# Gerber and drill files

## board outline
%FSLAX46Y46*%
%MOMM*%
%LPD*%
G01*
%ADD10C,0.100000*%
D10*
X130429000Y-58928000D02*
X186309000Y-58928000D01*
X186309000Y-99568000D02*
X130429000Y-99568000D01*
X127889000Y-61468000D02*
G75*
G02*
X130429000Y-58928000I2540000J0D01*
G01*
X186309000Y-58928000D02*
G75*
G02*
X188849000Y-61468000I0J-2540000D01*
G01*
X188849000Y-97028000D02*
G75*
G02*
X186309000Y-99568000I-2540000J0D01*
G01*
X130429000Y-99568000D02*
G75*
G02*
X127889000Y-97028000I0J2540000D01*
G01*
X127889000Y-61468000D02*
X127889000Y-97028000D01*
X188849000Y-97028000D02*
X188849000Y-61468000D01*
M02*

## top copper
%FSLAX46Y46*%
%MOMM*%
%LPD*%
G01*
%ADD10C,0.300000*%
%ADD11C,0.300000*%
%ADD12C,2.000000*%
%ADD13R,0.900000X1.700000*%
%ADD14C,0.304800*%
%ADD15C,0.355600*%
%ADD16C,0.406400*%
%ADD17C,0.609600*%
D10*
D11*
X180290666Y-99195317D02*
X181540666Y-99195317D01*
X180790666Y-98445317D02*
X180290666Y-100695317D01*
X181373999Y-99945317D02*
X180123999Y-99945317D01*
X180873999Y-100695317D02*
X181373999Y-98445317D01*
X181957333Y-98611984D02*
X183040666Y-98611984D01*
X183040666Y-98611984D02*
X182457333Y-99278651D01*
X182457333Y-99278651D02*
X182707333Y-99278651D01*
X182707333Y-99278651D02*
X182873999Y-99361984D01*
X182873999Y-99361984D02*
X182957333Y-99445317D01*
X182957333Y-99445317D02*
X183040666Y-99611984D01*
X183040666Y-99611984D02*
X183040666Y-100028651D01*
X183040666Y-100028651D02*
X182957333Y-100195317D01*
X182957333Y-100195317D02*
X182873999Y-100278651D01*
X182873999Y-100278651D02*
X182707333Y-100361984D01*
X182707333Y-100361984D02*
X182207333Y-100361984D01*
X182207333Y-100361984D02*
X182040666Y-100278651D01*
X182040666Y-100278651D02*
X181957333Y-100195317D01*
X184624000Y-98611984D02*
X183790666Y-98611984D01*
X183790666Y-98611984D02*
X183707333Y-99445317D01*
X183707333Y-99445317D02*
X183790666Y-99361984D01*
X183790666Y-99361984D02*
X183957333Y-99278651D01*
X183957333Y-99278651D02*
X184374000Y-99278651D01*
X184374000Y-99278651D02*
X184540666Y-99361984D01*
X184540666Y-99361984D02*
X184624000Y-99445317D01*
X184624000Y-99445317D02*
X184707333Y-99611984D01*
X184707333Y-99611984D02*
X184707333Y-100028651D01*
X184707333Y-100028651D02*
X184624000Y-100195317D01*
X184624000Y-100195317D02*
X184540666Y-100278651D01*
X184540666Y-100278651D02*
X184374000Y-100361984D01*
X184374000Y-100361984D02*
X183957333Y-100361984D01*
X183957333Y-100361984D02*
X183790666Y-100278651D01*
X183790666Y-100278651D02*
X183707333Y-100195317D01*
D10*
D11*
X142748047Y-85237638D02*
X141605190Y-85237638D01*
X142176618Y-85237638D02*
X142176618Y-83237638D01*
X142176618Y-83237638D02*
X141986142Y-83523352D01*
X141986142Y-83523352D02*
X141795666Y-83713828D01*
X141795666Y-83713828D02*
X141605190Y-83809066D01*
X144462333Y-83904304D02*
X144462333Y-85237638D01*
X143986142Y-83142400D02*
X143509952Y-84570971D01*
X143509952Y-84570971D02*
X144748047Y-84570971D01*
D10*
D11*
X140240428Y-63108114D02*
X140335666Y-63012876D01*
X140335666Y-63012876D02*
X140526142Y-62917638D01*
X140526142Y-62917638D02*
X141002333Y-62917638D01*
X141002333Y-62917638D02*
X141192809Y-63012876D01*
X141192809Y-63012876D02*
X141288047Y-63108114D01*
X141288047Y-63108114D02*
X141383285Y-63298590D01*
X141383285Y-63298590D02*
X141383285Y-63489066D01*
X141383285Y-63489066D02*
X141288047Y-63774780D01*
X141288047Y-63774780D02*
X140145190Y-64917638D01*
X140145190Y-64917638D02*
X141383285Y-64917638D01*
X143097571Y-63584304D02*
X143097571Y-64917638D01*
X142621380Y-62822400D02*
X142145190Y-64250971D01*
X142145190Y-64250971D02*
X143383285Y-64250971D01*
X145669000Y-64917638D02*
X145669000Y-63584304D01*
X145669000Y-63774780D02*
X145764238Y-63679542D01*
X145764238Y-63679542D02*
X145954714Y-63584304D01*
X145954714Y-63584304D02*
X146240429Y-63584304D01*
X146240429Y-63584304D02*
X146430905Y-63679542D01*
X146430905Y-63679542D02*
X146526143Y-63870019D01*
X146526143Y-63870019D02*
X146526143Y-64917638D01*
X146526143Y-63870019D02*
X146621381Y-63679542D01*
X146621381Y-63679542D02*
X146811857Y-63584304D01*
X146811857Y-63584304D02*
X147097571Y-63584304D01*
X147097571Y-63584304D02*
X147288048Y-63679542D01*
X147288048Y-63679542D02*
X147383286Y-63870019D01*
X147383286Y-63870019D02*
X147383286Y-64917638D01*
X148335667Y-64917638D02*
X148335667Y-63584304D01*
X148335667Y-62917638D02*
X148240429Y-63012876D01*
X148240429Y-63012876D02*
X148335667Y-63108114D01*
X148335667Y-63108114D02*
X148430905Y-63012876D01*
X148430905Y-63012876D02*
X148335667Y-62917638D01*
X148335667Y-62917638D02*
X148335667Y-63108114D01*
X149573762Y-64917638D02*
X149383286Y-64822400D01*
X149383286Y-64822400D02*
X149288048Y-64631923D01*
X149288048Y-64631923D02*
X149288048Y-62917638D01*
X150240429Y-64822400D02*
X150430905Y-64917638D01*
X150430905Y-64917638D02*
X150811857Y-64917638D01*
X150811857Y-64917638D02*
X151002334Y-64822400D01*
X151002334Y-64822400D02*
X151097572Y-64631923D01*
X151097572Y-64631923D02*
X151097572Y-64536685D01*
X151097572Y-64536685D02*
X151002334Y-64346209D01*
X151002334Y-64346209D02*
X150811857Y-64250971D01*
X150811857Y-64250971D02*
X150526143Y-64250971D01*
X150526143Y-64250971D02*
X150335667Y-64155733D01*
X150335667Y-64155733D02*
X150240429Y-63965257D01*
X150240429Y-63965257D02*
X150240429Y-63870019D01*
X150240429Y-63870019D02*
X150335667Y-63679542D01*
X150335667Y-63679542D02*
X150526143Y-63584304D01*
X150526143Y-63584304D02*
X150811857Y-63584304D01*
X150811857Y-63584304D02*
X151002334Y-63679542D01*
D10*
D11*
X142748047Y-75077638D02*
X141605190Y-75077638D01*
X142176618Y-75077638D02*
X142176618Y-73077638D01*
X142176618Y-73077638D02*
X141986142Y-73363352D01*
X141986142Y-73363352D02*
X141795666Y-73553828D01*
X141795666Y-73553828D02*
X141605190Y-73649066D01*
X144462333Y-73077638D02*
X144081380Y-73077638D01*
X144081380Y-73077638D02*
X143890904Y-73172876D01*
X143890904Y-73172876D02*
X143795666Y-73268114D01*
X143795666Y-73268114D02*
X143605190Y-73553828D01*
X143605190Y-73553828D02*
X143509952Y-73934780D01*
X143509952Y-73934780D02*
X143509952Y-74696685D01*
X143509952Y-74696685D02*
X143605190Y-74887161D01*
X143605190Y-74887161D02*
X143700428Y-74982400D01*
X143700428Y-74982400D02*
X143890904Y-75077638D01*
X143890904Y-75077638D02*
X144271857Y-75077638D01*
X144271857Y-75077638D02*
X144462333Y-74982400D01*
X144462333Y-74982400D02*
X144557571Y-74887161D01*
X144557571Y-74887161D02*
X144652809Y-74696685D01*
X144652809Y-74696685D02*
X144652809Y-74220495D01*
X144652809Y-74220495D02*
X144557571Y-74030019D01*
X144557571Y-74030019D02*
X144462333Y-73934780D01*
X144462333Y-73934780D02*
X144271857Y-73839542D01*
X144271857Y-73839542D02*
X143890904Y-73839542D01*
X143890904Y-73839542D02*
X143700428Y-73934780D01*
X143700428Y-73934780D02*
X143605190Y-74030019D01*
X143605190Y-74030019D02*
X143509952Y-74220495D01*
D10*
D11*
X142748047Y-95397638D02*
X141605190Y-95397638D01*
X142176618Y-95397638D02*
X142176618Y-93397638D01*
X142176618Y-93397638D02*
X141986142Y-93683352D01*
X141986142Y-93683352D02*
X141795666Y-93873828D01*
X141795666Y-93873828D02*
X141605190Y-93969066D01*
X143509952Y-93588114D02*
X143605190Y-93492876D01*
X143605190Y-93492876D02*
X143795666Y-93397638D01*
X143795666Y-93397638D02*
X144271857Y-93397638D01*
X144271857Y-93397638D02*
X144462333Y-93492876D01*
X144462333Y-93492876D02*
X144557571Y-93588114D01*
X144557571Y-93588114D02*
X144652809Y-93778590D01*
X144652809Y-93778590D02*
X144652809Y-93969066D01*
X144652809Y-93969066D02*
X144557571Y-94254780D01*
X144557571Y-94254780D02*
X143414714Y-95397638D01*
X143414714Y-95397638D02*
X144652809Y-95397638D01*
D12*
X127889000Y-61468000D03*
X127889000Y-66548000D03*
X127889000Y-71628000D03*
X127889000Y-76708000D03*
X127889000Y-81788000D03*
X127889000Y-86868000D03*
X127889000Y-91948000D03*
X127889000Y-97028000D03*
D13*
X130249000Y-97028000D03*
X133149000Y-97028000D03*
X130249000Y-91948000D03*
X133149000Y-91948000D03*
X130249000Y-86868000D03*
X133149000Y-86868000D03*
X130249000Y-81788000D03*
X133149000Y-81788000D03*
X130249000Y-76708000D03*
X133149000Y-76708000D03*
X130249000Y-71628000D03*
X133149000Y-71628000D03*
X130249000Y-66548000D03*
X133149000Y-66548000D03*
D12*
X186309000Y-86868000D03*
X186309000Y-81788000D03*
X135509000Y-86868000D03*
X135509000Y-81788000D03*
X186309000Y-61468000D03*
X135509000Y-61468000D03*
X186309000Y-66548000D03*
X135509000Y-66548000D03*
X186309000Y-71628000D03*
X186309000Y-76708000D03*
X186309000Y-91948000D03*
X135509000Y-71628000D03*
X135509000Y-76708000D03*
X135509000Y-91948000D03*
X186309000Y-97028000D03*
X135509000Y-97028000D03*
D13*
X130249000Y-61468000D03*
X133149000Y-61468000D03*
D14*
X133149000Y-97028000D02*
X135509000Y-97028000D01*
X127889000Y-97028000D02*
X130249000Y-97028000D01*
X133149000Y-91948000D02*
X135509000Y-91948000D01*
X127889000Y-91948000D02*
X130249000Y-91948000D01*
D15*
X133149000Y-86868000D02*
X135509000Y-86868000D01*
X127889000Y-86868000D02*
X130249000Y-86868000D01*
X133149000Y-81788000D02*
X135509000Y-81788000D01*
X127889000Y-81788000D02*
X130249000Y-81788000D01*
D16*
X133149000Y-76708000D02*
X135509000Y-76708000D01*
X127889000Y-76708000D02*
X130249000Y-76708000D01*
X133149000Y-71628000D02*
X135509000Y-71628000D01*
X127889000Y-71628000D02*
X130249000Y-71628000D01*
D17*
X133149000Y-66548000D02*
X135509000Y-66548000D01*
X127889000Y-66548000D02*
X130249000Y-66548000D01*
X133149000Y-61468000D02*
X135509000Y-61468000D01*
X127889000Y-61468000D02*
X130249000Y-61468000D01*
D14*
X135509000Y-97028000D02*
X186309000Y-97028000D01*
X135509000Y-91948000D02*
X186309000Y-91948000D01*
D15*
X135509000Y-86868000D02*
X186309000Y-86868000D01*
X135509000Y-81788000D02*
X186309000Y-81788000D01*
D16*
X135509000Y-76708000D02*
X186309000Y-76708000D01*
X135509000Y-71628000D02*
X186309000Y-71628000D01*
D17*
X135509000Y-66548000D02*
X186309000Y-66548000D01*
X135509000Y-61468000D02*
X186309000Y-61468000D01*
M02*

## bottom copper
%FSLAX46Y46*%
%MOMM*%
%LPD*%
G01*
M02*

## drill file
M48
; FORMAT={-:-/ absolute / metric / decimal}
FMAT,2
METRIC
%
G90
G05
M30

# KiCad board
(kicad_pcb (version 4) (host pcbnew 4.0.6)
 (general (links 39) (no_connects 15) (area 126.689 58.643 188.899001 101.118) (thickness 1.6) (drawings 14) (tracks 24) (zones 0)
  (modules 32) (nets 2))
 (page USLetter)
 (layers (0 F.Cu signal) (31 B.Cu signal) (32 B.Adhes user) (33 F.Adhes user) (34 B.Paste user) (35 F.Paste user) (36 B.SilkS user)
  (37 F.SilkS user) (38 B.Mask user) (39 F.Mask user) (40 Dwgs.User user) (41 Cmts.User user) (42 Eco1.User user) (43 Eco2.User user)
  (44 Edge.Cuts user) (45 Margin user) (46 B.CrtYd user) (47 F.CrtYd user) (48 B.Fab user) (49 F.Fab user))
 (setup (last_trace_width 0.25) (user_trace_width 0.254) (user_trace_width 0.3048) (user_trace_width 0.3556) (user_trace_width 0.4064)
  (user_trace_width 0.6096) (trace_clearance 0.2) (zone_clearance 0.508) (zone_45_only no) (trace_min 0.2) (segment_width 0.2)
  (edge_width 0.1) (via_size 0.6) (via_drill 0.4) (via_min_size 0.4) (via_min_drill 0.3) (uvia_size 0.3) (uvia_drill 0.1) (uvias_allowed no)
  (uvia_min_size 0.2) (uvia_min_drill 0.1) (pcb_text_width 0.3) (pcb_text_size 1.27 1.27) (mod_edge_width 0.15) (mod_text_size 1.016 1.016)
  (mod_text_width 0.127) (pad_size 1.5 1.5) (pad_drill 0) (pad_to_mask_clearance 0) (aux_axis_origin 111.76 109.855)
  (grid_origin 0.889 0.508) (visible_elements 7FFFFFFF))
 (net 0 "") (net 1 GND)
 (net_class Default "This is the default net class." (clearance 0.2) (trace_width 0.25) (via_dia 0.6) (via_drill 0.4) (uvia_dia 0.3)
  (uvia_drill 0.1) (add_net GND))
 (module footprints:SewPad (layer F.Cu) (at 127.889 61.468 90)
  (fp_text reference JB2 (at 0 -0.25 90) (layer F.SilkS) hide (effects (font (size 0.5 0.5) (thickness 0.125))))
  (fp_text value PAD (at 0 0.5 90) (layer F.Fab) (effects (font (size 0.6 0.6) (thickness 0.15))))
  (pad 1 smd circle (at 0 0 90) (size 2 2) (layers F.Cu F.Mask) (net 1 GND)))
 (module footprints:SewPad (layer F.Cu) (at 127.889 66.548 90)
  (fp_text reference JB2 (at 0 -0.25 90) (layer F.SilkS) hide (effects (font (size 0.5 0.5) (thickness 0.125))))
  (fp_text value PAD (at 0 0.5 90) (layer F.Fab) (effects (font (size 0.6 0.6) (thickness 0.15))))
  (pad 1 smd circle (at 0 0 90) (size 2 2) (layers F.Cu F.Mask) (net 1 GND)))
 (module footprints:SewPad (layer F.Cu) (at 127.889 71.628 90)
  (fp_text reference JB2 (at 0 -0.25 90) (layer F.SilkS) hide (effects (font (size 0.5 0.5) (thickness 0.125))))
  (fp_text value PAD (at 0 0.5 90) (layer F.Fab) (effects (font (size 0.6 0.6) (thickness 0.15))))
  (pad 1 smd circle (at 0 0 90) (size 2 2) (layers F.Cu F.Mask) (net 1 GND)))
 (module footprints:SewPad (layer F.Cu) (at 127.889 76.708 90)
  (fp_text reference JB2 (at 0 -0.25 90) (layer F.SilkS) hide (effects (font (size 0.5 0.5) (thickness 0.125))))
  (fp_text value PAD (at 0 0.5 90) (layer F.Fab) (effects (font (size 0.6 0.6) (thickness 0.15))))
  (pad 1 smd circle (at 0 0 90) (size 2 2) (layers F.Cu F.Mask) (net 1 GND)))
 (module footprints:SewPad (layer F.Cu) (at 127.889 81.788 90)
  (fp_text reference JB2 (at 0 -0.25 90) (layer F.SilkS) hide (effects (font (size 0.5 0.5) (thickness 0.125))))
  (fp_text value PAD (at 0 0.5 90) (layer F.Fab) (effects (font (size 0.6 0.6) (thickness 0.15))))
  (pad 1 smd circle (at 0 0 90) (size 2 2) (layers F.Cu F.Mask) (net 1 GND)))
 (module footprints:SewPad (layer F.Cu) (at 127.889 86.868 90)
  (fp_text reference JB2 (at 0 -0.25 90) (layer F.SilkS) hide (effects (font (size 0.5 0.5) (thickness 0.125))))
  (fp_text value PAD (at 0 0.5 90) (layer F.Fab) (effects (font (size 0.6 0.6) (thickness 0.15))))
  (pad 1 smd circle (at 0 0 90) (size 2 2) (layers F.Cu F.Mask) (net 1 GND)))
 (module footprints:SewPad (layer F.Cu) (at 127.889 91.948 90)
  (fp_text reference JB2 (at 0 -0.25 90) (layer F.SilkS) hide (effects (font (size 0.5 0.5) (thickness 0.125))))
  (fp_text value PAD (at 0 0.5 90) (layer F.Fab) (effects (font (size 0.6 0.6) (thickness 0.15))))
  (pad 1 smd circle (at 0 0 90) (size 2 2) (layers F.Cu F.Mask) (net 1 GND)))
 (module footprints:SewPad (layer F.Cu) (at 127.889 97.028 90)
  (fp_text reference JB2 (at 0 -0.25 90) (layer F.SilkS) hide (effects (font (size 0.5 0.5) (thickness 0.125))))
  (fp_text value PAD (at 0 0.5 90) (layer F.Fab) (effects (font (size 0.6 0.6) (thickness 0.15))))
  (pad 1 smd circle (at 0 0 90) (size 2 2) (layers F.Cu F.Mask) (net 1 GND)))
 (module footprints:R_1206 (layer F.Cu) (at 131.699 97.028)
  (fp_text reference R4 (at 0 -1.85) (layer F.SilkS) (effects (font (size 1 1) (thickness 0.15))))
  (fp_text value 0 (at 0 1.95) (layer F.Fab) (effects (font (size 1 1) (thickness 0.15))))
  (pad 1 smd rect (at -1.45 0) (size 0.9 1.7) (layers F.Cu F.Paste F.Mask) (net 1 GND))
  (pad 2 smd rect (at 1.45 0) (size 0.9 1.7) (layers F.Cu F.Paste F.Mask) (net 1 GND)))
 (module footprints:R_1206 (layer F.Cu) (at 131.699 91.948)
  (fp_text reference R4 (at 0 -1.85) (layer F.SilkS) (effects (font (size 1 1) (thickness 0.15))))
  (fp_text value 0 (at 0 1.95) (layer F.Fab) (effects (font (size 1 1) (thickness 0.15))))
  (pad 1 smd rect (at -1.45 0) (size 0.9 1.7) (layers F.Cu F.Paste F.Mask) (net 1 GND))
  (pad 2 smd rect (at 1.45 0) (size 0.9 1.7) (layers F.Cu F.Paste F.Mask) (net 1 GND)))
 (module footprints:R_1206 (layer F.Cu) (at 131.699 86.868)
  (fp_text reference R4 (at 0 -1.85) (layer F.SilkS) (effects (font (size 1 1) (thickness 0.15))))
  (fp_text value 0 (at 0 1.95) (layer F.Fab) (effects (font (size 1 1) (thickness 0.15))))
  (pad 1 smd rect (at -1.45 0) (size 0.9 1.7) (layers F.Cu F.Paste F.Mask) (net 1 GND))
  (pad 2 smd rect (at 1.45 0) (size 0.9 1.7) (layers F.Cu F.Paste F.Mask) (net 1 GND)))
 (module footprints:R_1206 (layer F.Cu) (at 131.699 81.788)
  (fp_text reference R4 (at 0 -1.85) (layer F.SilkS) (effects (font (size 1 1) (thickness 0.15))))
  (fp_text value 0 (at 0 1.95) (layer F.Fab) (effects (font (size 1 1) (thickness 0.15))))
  (pad 1 smd rect (at -1.45 0) (size 0.9 1.7) (layers F.Cu F.Paste F.Mask) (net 1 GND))
  (pad 2 smd rect (at 1.45 0) (size 0.9 1.7) (layers F.Cu F.Paste F.Mask) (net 1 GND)))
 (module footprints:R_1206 (layer F.Cu) (at 131.699 76.708)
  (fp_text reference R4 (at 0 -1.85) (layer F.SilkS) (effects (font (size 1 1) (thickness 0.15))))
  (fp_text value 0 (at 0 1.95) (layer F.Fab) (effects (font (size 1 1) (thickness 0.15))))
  (pad 1 smd rect (at -1.45 0) (size 0.9 1.7) (layers F.Cu F.Paste F.Mask) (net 1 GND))
  (pad 2 smd rect (at 1.45 0) (size 0.9 1.7) (layers F.Cu F.Paste F.Mask) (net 1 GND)))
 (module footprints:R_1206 (layer F.Cu) (at 131.699 71.628)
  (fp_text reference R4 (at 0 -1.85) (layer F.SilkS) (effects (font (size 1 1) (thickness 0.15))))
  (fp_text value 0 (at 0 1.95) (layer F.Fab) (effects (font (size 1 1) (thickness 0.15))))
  (pad 1 smd rect (at -1.45 0) (size 0.9 1.7) (layers F.Cu F.Paste F.Mask) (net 1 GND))
  (pad 2 smd rect (at 1.45 0) (size 0.9 1.7) (layers F.Cu F.Paste F.Mask) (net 1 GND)))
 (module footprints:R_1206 (layer F.Cu) (at 131.699 66.548)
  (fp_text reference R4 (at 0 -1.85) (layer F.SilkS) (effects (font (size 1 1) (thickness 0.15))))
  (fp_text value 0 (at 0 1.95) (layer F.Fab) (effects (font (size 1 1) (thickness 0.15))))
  (pad 1 smd rect (at -1.45 0) (size 0.9 1.7) (layers F.Cu F.Paste F.Mask) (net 1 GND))
  (pad 2 smd rect (at 1.45 0) (size 0.9 1.7) (layers F.Cu F.Paste F.Mask) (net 1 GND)))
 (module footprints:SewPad (layer F.Cu) (at 186.309 86.868 90)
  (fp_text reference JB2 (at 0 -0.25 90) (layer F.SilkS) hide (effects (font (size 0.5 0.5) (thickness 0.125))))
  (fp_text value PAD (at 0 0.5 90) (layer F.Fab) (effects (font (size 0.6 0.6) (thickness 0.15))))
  (pad 1 smd circle (at 0 0 90) (size 2 2) (layers F.Cu F.Mask) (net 1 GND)))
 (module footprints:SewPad (layer F.Cu) (at 186.309 81.788 90)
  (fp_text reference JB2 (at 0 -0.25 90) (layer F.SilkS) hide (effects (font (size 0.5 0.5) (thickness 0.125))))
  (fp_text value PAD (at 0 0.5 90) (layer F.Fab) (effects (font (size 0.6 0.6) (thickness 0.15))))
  (pad 1 smd circle (at 0 0 90) (size 2 2) (layers F.Cu F.Mask) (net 1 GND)))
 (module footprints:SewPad (layer F.Cu) (at 135.509 86.868 90)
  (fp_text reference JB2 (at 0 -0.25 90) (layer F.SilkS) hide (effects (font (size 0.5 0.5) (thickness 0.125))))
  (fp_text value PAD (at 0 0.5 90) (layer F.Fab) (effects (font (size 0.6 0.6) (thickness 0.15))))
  (pad 1 smd circle (at 0 0 90) (size 2 2) (layers F.Cu F.Mask) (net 1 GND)))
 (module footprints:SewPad (layer F.Cu) (at 135.509 81.788 90)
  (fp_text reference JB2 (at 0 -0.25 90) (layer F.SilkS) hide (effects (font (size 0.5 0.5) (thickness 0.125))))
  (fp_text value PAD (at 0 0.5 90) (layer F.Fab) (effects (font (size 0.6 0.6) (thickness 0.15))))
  (pad 1 smd circle (at 0 0 90) (size 2 2) (layers F.Cu F.Mask) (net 1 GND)))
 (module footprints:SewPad (layer F.Cu) (at 186.309 61.468 90)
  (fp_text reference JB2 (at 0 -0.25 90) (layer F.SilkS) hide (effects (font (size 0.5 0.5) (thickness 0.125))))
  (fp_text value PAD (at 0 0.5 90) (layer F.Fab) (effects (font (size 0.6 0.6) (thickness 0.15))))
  (pad 1 smd circle (at 0 0 90) (size 2 2) (layers F.Cu F.Mask) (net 1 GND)))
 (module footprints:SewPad (layer F.Cu) (at 135.509 61.468 90)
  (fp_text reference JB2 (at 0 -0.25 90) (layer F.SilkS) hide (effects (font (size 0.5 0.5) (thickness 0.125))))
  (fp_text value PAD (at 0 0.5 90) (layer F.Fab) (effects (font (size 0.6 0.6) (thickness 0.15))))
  (pad 1 smd circle (at 0 0 90) (size 2 2) (layers F.Cu F.Mask) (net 1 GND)))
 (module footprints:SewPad (layer F.Cu) (at 186.309 66.548 90)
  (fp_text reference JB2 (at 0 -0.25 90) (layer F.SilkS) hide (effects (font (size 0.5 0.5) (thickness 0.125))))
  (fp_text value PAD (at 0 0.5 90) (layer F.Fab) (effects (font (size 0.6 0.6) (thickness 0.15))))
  (pad 1 smd circle (at 0 0 90) (size 2 2) (layers F.Cu F.Mask) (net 1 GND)))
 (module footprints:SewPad (layer F.Cu) (at 135.509 66.548 90)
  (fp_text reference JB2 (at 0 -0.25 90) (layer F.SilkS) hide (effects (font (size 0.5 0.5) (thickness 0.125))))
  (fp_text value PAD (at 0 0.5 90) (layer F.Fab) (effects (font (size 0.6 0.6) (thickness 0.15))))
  (pad 1 smd circle (at 0 0 90) (size 2 2) (layers F.Cu F.Mask) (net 1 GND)))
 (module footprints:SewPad (layer F.Cu) (at 186.309 71.628 90)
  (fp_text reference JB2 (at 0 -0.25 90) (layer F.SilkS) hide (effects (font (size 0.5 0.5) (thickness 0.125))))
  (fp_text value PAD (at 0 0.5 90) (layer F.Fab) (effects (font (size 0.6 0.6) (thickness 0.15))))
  (pad 1 smd circle (at 0 0 90) (size 2 2) (layers F.Cu F.Mask) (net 1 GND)))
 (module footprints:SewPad (layer F.Cu) (at 186.309 76.708 90)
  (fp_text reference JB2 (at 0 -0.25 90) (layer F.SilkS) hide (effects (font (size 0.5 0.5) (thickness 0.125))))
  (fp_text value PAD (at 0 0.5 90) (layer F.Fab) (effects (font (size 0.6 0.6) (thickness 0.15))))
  (pad 1 smd circle (at 0 0 90) (size 2 2) (layers F.Cu F.Mask) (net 1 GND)))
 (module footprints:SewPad (layer F.Cu) (at 186.309 91.948 90)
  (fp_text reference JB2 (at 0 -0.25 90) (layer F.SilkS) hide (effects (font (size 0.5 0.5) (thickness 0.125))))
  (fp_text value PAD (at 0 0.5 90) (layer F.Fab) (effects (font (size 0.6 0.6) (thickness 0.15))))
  (pad 1 smd circle (at 0 0 90) (size 2 2) (layers F.Cu F.Mask) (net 1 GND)))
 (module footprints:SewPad (layer F.Cu) (at 135.509 71.628 90)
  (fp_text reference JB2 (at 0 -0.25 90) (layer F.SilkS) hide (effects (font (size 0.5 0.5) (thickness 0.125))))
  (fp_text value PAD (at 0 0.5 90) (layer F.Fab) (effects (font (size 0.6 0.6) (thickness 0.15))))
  (pad 1 smd circle (at 0 0 90) (size 2 2) (layers F.Cu F.Mask) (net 1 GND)))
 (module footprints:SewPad (layer F.Cu) (at 135.509 76.708 90)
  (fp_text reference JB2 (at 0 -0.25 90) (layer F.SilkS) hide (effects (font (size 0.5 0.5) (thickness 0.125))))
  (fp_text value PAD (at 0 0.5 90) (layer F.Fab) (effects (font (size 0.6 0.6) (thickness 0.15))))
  (pad 1 smd circle (at 0 0 90) (size 2 2) (layers F.Cu F.Mask) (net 1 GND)))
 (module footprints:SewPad (layer F.Cu) (at 135.509 91.948 90)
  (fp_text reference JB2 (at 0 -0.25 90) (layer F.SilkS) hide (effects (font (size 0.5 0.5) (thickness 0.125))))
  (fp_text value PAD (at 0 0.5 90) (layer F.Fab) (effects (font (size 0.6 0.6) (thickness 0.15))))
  (pad 1 smd circle (at 0 0 90) (size 2 2) (layers F.Cu F.Mask) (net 1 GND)))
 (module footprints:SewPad (layer F.Cu) (at 186.309 97.028 90)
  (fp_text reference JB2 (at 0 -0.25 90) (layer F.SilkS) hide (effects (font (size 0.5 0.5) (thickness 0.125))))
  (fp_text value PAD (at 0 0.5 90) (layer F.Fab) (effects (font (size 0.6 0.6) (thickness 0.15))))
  (pad 1 smd circle (at 0 0 90) (size 2 2) (layers F.Cu F.Mask) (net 1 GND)))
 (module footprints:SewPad (layer F.Cu) (at 135.509 97.028 90)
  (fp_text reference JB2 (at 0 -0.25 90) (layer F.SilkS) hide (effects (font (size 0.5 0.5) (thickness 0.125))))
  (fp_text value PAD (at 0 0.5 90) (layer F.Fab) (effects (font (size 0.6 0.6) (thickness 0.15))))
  (pad 1 smd circle (at 0 0 90) (size 2 2) (layers F.Cu F.Mask) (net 1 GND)))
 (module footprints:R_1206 (layer F.Cu) (at 131.699 61.468)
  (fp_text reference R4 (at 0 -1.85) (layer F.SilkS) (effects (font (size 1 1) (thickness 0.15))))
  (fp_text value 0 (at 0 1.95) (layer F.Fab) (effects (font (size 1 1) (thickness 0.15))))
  (pad 1 smd rect (at -1.45 0) (size 0.9 1.7) (layers F.Cu F.Paste F.Mask) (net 1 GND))
  (pad 2 smd rect (at 1.45 0) (size 0.9 1.7) (layers F.Cu F.Paste F.Mask) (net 1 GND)))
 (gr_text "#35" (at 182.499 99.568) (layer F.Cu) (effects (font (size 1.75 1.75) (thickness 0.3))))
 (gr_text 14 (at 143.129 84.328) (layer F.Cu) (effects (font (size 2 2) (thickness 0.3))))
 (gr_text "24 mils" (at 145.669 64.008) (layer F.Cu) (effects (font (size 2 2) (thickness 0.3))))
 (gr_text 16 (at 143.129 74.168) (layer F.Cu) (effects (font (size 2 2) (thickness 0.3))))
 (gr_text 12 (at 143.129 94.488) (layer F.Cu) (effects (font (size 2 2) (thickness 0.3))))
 (gr_line (start 130.429 58.928) (end 186.309 58.928) (angle 90) (layer Edge.Cuts) (width 0.1))
 (gr_line (start 186.309 99.568) (end 130.429 99.568) (angle 90) (layer Edge.Cuts) (width 0.1))
 (gr_arc (start 130.429 61.468) (end 127.889 61.468) (angle 90) (layer Edge.Cuts) (width 0.1))
 (gr_arc (start 186.309 61.468) (end 186.309 58.928) (angle 90) (layer Edge.Cuts) (width 0.1))
 (gr_arc (start 186.309 97.028) (end 188.849 97.028) (angle 90) (layer Edge.Cuts) (width 0.1))
 (gr_arc (start 130.429 97.028) (end 130.429 99.568) (angle 90) (layer Edge.Cuts) (width 0.1))
 (gr_line (start 127.889 61.468) (end 127.889 97.028) (angle 90) (layer Edge.Cuts) (width 0.1))
 (gr_line (start 188.849 97.028) (end 188.849 61.468) (angle 90) (layer Edge.Cuts) (width 0.1))
 (segment (start 133.149 97.028) (end 135.509 97.028) (width 0.3048) (layer F.Cu) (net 1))
 (segment (start 127.889 97.028) (end 130.249 97.028) (width 0.3048) (layer F.Cu) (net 1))
 (segment (start 133.149 91.948) (end 135.509 91.948) (width 0.3048) (layer F.Cu) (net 1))
 (segment (start 127.889 91.948) (end 130.249 91.948) (width 0.3048) (layer F.Cu) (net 1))
 (segment (start 133.149 86.868) (end 135.509 86.868) (width 0.3556) (layer F.Cu) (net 1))
 (segment (start 127.889 86.868) (end 130.249 86.868) (width 0.3556) (layer F.Cu) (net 1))
 (segment (start 133.149 81.788) (end 135.509 81.788) (width 0.3556) (layer F.Cu) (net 1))
 (segment (start 127.889 81.788) (end 130.249 81.788) (width 0.3556) (layer F.Cu) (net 1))
 (segment (start 133.149 76.708) (end 135.509 76.708) (width 0.4064) (layer F.Cu) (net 1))
 (segment (start 127.889 76.708) (end 130.249 76.708) (width 0.4064) (layer F.Cu) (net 1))
 (segment (start 133.149 71.628) (end 135.509 71.628) (width 0.4064) (layer F.Cu) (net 1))
 (segment (start 127.889 71.628) (end 130.249 71.628) (width 0.4064) (layer F.Cu) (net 1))
 (segment (start 133.149 66.548) (end 135.509 66.548) (width 0.6096) (layer F.Cu) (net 1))
 (segment (start 127.889 66.548) (end 130.249 66.548) (width 0.6096) (layer F.Cu) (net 1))
 (segment (start 133.149 61.468) (end 135.509 61.468) (width 0.6096) (layer F.Cu) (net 1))
 (segment (start 127.889 61.468) (end 130.249 61.468) (width 0.6096) (layer F.Cu) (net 1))
 (segment (start 135.509 97.028) (end 186.309 97.028) (width 0.3048) (layer F.Cu) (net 1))
 (segment (start 135.509 91.948) (end 186.309 91.948) (width 0.3048) (layer F.Cu) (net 1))
 (segment (start 135.509 86.868) (end 186.309 86.868) (width 0.3556) (layer F.Cu) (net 1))
 (segment (start 135.509 81.788) (end 186.309 81.788) (width 0.3556) (layer F.Cu) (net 1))
 (segment (start 135.509 76.708) (end 186.309 76.708) (width 0.4064) (layer F.Cu) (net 1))
 (segment (start 135.509 71.628) (end 186.309 71.628) (width 0.4064) (layer F.Cu) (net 1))
 (segment (start 135.509 66.548) (end 186.309 66.548) (width 0.6096) (layer F.Cu) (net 1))
 (segment (start 135.509 61.468) (end 186.309 61.468) (width 0.6096) (layer F.Cu) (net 1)))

